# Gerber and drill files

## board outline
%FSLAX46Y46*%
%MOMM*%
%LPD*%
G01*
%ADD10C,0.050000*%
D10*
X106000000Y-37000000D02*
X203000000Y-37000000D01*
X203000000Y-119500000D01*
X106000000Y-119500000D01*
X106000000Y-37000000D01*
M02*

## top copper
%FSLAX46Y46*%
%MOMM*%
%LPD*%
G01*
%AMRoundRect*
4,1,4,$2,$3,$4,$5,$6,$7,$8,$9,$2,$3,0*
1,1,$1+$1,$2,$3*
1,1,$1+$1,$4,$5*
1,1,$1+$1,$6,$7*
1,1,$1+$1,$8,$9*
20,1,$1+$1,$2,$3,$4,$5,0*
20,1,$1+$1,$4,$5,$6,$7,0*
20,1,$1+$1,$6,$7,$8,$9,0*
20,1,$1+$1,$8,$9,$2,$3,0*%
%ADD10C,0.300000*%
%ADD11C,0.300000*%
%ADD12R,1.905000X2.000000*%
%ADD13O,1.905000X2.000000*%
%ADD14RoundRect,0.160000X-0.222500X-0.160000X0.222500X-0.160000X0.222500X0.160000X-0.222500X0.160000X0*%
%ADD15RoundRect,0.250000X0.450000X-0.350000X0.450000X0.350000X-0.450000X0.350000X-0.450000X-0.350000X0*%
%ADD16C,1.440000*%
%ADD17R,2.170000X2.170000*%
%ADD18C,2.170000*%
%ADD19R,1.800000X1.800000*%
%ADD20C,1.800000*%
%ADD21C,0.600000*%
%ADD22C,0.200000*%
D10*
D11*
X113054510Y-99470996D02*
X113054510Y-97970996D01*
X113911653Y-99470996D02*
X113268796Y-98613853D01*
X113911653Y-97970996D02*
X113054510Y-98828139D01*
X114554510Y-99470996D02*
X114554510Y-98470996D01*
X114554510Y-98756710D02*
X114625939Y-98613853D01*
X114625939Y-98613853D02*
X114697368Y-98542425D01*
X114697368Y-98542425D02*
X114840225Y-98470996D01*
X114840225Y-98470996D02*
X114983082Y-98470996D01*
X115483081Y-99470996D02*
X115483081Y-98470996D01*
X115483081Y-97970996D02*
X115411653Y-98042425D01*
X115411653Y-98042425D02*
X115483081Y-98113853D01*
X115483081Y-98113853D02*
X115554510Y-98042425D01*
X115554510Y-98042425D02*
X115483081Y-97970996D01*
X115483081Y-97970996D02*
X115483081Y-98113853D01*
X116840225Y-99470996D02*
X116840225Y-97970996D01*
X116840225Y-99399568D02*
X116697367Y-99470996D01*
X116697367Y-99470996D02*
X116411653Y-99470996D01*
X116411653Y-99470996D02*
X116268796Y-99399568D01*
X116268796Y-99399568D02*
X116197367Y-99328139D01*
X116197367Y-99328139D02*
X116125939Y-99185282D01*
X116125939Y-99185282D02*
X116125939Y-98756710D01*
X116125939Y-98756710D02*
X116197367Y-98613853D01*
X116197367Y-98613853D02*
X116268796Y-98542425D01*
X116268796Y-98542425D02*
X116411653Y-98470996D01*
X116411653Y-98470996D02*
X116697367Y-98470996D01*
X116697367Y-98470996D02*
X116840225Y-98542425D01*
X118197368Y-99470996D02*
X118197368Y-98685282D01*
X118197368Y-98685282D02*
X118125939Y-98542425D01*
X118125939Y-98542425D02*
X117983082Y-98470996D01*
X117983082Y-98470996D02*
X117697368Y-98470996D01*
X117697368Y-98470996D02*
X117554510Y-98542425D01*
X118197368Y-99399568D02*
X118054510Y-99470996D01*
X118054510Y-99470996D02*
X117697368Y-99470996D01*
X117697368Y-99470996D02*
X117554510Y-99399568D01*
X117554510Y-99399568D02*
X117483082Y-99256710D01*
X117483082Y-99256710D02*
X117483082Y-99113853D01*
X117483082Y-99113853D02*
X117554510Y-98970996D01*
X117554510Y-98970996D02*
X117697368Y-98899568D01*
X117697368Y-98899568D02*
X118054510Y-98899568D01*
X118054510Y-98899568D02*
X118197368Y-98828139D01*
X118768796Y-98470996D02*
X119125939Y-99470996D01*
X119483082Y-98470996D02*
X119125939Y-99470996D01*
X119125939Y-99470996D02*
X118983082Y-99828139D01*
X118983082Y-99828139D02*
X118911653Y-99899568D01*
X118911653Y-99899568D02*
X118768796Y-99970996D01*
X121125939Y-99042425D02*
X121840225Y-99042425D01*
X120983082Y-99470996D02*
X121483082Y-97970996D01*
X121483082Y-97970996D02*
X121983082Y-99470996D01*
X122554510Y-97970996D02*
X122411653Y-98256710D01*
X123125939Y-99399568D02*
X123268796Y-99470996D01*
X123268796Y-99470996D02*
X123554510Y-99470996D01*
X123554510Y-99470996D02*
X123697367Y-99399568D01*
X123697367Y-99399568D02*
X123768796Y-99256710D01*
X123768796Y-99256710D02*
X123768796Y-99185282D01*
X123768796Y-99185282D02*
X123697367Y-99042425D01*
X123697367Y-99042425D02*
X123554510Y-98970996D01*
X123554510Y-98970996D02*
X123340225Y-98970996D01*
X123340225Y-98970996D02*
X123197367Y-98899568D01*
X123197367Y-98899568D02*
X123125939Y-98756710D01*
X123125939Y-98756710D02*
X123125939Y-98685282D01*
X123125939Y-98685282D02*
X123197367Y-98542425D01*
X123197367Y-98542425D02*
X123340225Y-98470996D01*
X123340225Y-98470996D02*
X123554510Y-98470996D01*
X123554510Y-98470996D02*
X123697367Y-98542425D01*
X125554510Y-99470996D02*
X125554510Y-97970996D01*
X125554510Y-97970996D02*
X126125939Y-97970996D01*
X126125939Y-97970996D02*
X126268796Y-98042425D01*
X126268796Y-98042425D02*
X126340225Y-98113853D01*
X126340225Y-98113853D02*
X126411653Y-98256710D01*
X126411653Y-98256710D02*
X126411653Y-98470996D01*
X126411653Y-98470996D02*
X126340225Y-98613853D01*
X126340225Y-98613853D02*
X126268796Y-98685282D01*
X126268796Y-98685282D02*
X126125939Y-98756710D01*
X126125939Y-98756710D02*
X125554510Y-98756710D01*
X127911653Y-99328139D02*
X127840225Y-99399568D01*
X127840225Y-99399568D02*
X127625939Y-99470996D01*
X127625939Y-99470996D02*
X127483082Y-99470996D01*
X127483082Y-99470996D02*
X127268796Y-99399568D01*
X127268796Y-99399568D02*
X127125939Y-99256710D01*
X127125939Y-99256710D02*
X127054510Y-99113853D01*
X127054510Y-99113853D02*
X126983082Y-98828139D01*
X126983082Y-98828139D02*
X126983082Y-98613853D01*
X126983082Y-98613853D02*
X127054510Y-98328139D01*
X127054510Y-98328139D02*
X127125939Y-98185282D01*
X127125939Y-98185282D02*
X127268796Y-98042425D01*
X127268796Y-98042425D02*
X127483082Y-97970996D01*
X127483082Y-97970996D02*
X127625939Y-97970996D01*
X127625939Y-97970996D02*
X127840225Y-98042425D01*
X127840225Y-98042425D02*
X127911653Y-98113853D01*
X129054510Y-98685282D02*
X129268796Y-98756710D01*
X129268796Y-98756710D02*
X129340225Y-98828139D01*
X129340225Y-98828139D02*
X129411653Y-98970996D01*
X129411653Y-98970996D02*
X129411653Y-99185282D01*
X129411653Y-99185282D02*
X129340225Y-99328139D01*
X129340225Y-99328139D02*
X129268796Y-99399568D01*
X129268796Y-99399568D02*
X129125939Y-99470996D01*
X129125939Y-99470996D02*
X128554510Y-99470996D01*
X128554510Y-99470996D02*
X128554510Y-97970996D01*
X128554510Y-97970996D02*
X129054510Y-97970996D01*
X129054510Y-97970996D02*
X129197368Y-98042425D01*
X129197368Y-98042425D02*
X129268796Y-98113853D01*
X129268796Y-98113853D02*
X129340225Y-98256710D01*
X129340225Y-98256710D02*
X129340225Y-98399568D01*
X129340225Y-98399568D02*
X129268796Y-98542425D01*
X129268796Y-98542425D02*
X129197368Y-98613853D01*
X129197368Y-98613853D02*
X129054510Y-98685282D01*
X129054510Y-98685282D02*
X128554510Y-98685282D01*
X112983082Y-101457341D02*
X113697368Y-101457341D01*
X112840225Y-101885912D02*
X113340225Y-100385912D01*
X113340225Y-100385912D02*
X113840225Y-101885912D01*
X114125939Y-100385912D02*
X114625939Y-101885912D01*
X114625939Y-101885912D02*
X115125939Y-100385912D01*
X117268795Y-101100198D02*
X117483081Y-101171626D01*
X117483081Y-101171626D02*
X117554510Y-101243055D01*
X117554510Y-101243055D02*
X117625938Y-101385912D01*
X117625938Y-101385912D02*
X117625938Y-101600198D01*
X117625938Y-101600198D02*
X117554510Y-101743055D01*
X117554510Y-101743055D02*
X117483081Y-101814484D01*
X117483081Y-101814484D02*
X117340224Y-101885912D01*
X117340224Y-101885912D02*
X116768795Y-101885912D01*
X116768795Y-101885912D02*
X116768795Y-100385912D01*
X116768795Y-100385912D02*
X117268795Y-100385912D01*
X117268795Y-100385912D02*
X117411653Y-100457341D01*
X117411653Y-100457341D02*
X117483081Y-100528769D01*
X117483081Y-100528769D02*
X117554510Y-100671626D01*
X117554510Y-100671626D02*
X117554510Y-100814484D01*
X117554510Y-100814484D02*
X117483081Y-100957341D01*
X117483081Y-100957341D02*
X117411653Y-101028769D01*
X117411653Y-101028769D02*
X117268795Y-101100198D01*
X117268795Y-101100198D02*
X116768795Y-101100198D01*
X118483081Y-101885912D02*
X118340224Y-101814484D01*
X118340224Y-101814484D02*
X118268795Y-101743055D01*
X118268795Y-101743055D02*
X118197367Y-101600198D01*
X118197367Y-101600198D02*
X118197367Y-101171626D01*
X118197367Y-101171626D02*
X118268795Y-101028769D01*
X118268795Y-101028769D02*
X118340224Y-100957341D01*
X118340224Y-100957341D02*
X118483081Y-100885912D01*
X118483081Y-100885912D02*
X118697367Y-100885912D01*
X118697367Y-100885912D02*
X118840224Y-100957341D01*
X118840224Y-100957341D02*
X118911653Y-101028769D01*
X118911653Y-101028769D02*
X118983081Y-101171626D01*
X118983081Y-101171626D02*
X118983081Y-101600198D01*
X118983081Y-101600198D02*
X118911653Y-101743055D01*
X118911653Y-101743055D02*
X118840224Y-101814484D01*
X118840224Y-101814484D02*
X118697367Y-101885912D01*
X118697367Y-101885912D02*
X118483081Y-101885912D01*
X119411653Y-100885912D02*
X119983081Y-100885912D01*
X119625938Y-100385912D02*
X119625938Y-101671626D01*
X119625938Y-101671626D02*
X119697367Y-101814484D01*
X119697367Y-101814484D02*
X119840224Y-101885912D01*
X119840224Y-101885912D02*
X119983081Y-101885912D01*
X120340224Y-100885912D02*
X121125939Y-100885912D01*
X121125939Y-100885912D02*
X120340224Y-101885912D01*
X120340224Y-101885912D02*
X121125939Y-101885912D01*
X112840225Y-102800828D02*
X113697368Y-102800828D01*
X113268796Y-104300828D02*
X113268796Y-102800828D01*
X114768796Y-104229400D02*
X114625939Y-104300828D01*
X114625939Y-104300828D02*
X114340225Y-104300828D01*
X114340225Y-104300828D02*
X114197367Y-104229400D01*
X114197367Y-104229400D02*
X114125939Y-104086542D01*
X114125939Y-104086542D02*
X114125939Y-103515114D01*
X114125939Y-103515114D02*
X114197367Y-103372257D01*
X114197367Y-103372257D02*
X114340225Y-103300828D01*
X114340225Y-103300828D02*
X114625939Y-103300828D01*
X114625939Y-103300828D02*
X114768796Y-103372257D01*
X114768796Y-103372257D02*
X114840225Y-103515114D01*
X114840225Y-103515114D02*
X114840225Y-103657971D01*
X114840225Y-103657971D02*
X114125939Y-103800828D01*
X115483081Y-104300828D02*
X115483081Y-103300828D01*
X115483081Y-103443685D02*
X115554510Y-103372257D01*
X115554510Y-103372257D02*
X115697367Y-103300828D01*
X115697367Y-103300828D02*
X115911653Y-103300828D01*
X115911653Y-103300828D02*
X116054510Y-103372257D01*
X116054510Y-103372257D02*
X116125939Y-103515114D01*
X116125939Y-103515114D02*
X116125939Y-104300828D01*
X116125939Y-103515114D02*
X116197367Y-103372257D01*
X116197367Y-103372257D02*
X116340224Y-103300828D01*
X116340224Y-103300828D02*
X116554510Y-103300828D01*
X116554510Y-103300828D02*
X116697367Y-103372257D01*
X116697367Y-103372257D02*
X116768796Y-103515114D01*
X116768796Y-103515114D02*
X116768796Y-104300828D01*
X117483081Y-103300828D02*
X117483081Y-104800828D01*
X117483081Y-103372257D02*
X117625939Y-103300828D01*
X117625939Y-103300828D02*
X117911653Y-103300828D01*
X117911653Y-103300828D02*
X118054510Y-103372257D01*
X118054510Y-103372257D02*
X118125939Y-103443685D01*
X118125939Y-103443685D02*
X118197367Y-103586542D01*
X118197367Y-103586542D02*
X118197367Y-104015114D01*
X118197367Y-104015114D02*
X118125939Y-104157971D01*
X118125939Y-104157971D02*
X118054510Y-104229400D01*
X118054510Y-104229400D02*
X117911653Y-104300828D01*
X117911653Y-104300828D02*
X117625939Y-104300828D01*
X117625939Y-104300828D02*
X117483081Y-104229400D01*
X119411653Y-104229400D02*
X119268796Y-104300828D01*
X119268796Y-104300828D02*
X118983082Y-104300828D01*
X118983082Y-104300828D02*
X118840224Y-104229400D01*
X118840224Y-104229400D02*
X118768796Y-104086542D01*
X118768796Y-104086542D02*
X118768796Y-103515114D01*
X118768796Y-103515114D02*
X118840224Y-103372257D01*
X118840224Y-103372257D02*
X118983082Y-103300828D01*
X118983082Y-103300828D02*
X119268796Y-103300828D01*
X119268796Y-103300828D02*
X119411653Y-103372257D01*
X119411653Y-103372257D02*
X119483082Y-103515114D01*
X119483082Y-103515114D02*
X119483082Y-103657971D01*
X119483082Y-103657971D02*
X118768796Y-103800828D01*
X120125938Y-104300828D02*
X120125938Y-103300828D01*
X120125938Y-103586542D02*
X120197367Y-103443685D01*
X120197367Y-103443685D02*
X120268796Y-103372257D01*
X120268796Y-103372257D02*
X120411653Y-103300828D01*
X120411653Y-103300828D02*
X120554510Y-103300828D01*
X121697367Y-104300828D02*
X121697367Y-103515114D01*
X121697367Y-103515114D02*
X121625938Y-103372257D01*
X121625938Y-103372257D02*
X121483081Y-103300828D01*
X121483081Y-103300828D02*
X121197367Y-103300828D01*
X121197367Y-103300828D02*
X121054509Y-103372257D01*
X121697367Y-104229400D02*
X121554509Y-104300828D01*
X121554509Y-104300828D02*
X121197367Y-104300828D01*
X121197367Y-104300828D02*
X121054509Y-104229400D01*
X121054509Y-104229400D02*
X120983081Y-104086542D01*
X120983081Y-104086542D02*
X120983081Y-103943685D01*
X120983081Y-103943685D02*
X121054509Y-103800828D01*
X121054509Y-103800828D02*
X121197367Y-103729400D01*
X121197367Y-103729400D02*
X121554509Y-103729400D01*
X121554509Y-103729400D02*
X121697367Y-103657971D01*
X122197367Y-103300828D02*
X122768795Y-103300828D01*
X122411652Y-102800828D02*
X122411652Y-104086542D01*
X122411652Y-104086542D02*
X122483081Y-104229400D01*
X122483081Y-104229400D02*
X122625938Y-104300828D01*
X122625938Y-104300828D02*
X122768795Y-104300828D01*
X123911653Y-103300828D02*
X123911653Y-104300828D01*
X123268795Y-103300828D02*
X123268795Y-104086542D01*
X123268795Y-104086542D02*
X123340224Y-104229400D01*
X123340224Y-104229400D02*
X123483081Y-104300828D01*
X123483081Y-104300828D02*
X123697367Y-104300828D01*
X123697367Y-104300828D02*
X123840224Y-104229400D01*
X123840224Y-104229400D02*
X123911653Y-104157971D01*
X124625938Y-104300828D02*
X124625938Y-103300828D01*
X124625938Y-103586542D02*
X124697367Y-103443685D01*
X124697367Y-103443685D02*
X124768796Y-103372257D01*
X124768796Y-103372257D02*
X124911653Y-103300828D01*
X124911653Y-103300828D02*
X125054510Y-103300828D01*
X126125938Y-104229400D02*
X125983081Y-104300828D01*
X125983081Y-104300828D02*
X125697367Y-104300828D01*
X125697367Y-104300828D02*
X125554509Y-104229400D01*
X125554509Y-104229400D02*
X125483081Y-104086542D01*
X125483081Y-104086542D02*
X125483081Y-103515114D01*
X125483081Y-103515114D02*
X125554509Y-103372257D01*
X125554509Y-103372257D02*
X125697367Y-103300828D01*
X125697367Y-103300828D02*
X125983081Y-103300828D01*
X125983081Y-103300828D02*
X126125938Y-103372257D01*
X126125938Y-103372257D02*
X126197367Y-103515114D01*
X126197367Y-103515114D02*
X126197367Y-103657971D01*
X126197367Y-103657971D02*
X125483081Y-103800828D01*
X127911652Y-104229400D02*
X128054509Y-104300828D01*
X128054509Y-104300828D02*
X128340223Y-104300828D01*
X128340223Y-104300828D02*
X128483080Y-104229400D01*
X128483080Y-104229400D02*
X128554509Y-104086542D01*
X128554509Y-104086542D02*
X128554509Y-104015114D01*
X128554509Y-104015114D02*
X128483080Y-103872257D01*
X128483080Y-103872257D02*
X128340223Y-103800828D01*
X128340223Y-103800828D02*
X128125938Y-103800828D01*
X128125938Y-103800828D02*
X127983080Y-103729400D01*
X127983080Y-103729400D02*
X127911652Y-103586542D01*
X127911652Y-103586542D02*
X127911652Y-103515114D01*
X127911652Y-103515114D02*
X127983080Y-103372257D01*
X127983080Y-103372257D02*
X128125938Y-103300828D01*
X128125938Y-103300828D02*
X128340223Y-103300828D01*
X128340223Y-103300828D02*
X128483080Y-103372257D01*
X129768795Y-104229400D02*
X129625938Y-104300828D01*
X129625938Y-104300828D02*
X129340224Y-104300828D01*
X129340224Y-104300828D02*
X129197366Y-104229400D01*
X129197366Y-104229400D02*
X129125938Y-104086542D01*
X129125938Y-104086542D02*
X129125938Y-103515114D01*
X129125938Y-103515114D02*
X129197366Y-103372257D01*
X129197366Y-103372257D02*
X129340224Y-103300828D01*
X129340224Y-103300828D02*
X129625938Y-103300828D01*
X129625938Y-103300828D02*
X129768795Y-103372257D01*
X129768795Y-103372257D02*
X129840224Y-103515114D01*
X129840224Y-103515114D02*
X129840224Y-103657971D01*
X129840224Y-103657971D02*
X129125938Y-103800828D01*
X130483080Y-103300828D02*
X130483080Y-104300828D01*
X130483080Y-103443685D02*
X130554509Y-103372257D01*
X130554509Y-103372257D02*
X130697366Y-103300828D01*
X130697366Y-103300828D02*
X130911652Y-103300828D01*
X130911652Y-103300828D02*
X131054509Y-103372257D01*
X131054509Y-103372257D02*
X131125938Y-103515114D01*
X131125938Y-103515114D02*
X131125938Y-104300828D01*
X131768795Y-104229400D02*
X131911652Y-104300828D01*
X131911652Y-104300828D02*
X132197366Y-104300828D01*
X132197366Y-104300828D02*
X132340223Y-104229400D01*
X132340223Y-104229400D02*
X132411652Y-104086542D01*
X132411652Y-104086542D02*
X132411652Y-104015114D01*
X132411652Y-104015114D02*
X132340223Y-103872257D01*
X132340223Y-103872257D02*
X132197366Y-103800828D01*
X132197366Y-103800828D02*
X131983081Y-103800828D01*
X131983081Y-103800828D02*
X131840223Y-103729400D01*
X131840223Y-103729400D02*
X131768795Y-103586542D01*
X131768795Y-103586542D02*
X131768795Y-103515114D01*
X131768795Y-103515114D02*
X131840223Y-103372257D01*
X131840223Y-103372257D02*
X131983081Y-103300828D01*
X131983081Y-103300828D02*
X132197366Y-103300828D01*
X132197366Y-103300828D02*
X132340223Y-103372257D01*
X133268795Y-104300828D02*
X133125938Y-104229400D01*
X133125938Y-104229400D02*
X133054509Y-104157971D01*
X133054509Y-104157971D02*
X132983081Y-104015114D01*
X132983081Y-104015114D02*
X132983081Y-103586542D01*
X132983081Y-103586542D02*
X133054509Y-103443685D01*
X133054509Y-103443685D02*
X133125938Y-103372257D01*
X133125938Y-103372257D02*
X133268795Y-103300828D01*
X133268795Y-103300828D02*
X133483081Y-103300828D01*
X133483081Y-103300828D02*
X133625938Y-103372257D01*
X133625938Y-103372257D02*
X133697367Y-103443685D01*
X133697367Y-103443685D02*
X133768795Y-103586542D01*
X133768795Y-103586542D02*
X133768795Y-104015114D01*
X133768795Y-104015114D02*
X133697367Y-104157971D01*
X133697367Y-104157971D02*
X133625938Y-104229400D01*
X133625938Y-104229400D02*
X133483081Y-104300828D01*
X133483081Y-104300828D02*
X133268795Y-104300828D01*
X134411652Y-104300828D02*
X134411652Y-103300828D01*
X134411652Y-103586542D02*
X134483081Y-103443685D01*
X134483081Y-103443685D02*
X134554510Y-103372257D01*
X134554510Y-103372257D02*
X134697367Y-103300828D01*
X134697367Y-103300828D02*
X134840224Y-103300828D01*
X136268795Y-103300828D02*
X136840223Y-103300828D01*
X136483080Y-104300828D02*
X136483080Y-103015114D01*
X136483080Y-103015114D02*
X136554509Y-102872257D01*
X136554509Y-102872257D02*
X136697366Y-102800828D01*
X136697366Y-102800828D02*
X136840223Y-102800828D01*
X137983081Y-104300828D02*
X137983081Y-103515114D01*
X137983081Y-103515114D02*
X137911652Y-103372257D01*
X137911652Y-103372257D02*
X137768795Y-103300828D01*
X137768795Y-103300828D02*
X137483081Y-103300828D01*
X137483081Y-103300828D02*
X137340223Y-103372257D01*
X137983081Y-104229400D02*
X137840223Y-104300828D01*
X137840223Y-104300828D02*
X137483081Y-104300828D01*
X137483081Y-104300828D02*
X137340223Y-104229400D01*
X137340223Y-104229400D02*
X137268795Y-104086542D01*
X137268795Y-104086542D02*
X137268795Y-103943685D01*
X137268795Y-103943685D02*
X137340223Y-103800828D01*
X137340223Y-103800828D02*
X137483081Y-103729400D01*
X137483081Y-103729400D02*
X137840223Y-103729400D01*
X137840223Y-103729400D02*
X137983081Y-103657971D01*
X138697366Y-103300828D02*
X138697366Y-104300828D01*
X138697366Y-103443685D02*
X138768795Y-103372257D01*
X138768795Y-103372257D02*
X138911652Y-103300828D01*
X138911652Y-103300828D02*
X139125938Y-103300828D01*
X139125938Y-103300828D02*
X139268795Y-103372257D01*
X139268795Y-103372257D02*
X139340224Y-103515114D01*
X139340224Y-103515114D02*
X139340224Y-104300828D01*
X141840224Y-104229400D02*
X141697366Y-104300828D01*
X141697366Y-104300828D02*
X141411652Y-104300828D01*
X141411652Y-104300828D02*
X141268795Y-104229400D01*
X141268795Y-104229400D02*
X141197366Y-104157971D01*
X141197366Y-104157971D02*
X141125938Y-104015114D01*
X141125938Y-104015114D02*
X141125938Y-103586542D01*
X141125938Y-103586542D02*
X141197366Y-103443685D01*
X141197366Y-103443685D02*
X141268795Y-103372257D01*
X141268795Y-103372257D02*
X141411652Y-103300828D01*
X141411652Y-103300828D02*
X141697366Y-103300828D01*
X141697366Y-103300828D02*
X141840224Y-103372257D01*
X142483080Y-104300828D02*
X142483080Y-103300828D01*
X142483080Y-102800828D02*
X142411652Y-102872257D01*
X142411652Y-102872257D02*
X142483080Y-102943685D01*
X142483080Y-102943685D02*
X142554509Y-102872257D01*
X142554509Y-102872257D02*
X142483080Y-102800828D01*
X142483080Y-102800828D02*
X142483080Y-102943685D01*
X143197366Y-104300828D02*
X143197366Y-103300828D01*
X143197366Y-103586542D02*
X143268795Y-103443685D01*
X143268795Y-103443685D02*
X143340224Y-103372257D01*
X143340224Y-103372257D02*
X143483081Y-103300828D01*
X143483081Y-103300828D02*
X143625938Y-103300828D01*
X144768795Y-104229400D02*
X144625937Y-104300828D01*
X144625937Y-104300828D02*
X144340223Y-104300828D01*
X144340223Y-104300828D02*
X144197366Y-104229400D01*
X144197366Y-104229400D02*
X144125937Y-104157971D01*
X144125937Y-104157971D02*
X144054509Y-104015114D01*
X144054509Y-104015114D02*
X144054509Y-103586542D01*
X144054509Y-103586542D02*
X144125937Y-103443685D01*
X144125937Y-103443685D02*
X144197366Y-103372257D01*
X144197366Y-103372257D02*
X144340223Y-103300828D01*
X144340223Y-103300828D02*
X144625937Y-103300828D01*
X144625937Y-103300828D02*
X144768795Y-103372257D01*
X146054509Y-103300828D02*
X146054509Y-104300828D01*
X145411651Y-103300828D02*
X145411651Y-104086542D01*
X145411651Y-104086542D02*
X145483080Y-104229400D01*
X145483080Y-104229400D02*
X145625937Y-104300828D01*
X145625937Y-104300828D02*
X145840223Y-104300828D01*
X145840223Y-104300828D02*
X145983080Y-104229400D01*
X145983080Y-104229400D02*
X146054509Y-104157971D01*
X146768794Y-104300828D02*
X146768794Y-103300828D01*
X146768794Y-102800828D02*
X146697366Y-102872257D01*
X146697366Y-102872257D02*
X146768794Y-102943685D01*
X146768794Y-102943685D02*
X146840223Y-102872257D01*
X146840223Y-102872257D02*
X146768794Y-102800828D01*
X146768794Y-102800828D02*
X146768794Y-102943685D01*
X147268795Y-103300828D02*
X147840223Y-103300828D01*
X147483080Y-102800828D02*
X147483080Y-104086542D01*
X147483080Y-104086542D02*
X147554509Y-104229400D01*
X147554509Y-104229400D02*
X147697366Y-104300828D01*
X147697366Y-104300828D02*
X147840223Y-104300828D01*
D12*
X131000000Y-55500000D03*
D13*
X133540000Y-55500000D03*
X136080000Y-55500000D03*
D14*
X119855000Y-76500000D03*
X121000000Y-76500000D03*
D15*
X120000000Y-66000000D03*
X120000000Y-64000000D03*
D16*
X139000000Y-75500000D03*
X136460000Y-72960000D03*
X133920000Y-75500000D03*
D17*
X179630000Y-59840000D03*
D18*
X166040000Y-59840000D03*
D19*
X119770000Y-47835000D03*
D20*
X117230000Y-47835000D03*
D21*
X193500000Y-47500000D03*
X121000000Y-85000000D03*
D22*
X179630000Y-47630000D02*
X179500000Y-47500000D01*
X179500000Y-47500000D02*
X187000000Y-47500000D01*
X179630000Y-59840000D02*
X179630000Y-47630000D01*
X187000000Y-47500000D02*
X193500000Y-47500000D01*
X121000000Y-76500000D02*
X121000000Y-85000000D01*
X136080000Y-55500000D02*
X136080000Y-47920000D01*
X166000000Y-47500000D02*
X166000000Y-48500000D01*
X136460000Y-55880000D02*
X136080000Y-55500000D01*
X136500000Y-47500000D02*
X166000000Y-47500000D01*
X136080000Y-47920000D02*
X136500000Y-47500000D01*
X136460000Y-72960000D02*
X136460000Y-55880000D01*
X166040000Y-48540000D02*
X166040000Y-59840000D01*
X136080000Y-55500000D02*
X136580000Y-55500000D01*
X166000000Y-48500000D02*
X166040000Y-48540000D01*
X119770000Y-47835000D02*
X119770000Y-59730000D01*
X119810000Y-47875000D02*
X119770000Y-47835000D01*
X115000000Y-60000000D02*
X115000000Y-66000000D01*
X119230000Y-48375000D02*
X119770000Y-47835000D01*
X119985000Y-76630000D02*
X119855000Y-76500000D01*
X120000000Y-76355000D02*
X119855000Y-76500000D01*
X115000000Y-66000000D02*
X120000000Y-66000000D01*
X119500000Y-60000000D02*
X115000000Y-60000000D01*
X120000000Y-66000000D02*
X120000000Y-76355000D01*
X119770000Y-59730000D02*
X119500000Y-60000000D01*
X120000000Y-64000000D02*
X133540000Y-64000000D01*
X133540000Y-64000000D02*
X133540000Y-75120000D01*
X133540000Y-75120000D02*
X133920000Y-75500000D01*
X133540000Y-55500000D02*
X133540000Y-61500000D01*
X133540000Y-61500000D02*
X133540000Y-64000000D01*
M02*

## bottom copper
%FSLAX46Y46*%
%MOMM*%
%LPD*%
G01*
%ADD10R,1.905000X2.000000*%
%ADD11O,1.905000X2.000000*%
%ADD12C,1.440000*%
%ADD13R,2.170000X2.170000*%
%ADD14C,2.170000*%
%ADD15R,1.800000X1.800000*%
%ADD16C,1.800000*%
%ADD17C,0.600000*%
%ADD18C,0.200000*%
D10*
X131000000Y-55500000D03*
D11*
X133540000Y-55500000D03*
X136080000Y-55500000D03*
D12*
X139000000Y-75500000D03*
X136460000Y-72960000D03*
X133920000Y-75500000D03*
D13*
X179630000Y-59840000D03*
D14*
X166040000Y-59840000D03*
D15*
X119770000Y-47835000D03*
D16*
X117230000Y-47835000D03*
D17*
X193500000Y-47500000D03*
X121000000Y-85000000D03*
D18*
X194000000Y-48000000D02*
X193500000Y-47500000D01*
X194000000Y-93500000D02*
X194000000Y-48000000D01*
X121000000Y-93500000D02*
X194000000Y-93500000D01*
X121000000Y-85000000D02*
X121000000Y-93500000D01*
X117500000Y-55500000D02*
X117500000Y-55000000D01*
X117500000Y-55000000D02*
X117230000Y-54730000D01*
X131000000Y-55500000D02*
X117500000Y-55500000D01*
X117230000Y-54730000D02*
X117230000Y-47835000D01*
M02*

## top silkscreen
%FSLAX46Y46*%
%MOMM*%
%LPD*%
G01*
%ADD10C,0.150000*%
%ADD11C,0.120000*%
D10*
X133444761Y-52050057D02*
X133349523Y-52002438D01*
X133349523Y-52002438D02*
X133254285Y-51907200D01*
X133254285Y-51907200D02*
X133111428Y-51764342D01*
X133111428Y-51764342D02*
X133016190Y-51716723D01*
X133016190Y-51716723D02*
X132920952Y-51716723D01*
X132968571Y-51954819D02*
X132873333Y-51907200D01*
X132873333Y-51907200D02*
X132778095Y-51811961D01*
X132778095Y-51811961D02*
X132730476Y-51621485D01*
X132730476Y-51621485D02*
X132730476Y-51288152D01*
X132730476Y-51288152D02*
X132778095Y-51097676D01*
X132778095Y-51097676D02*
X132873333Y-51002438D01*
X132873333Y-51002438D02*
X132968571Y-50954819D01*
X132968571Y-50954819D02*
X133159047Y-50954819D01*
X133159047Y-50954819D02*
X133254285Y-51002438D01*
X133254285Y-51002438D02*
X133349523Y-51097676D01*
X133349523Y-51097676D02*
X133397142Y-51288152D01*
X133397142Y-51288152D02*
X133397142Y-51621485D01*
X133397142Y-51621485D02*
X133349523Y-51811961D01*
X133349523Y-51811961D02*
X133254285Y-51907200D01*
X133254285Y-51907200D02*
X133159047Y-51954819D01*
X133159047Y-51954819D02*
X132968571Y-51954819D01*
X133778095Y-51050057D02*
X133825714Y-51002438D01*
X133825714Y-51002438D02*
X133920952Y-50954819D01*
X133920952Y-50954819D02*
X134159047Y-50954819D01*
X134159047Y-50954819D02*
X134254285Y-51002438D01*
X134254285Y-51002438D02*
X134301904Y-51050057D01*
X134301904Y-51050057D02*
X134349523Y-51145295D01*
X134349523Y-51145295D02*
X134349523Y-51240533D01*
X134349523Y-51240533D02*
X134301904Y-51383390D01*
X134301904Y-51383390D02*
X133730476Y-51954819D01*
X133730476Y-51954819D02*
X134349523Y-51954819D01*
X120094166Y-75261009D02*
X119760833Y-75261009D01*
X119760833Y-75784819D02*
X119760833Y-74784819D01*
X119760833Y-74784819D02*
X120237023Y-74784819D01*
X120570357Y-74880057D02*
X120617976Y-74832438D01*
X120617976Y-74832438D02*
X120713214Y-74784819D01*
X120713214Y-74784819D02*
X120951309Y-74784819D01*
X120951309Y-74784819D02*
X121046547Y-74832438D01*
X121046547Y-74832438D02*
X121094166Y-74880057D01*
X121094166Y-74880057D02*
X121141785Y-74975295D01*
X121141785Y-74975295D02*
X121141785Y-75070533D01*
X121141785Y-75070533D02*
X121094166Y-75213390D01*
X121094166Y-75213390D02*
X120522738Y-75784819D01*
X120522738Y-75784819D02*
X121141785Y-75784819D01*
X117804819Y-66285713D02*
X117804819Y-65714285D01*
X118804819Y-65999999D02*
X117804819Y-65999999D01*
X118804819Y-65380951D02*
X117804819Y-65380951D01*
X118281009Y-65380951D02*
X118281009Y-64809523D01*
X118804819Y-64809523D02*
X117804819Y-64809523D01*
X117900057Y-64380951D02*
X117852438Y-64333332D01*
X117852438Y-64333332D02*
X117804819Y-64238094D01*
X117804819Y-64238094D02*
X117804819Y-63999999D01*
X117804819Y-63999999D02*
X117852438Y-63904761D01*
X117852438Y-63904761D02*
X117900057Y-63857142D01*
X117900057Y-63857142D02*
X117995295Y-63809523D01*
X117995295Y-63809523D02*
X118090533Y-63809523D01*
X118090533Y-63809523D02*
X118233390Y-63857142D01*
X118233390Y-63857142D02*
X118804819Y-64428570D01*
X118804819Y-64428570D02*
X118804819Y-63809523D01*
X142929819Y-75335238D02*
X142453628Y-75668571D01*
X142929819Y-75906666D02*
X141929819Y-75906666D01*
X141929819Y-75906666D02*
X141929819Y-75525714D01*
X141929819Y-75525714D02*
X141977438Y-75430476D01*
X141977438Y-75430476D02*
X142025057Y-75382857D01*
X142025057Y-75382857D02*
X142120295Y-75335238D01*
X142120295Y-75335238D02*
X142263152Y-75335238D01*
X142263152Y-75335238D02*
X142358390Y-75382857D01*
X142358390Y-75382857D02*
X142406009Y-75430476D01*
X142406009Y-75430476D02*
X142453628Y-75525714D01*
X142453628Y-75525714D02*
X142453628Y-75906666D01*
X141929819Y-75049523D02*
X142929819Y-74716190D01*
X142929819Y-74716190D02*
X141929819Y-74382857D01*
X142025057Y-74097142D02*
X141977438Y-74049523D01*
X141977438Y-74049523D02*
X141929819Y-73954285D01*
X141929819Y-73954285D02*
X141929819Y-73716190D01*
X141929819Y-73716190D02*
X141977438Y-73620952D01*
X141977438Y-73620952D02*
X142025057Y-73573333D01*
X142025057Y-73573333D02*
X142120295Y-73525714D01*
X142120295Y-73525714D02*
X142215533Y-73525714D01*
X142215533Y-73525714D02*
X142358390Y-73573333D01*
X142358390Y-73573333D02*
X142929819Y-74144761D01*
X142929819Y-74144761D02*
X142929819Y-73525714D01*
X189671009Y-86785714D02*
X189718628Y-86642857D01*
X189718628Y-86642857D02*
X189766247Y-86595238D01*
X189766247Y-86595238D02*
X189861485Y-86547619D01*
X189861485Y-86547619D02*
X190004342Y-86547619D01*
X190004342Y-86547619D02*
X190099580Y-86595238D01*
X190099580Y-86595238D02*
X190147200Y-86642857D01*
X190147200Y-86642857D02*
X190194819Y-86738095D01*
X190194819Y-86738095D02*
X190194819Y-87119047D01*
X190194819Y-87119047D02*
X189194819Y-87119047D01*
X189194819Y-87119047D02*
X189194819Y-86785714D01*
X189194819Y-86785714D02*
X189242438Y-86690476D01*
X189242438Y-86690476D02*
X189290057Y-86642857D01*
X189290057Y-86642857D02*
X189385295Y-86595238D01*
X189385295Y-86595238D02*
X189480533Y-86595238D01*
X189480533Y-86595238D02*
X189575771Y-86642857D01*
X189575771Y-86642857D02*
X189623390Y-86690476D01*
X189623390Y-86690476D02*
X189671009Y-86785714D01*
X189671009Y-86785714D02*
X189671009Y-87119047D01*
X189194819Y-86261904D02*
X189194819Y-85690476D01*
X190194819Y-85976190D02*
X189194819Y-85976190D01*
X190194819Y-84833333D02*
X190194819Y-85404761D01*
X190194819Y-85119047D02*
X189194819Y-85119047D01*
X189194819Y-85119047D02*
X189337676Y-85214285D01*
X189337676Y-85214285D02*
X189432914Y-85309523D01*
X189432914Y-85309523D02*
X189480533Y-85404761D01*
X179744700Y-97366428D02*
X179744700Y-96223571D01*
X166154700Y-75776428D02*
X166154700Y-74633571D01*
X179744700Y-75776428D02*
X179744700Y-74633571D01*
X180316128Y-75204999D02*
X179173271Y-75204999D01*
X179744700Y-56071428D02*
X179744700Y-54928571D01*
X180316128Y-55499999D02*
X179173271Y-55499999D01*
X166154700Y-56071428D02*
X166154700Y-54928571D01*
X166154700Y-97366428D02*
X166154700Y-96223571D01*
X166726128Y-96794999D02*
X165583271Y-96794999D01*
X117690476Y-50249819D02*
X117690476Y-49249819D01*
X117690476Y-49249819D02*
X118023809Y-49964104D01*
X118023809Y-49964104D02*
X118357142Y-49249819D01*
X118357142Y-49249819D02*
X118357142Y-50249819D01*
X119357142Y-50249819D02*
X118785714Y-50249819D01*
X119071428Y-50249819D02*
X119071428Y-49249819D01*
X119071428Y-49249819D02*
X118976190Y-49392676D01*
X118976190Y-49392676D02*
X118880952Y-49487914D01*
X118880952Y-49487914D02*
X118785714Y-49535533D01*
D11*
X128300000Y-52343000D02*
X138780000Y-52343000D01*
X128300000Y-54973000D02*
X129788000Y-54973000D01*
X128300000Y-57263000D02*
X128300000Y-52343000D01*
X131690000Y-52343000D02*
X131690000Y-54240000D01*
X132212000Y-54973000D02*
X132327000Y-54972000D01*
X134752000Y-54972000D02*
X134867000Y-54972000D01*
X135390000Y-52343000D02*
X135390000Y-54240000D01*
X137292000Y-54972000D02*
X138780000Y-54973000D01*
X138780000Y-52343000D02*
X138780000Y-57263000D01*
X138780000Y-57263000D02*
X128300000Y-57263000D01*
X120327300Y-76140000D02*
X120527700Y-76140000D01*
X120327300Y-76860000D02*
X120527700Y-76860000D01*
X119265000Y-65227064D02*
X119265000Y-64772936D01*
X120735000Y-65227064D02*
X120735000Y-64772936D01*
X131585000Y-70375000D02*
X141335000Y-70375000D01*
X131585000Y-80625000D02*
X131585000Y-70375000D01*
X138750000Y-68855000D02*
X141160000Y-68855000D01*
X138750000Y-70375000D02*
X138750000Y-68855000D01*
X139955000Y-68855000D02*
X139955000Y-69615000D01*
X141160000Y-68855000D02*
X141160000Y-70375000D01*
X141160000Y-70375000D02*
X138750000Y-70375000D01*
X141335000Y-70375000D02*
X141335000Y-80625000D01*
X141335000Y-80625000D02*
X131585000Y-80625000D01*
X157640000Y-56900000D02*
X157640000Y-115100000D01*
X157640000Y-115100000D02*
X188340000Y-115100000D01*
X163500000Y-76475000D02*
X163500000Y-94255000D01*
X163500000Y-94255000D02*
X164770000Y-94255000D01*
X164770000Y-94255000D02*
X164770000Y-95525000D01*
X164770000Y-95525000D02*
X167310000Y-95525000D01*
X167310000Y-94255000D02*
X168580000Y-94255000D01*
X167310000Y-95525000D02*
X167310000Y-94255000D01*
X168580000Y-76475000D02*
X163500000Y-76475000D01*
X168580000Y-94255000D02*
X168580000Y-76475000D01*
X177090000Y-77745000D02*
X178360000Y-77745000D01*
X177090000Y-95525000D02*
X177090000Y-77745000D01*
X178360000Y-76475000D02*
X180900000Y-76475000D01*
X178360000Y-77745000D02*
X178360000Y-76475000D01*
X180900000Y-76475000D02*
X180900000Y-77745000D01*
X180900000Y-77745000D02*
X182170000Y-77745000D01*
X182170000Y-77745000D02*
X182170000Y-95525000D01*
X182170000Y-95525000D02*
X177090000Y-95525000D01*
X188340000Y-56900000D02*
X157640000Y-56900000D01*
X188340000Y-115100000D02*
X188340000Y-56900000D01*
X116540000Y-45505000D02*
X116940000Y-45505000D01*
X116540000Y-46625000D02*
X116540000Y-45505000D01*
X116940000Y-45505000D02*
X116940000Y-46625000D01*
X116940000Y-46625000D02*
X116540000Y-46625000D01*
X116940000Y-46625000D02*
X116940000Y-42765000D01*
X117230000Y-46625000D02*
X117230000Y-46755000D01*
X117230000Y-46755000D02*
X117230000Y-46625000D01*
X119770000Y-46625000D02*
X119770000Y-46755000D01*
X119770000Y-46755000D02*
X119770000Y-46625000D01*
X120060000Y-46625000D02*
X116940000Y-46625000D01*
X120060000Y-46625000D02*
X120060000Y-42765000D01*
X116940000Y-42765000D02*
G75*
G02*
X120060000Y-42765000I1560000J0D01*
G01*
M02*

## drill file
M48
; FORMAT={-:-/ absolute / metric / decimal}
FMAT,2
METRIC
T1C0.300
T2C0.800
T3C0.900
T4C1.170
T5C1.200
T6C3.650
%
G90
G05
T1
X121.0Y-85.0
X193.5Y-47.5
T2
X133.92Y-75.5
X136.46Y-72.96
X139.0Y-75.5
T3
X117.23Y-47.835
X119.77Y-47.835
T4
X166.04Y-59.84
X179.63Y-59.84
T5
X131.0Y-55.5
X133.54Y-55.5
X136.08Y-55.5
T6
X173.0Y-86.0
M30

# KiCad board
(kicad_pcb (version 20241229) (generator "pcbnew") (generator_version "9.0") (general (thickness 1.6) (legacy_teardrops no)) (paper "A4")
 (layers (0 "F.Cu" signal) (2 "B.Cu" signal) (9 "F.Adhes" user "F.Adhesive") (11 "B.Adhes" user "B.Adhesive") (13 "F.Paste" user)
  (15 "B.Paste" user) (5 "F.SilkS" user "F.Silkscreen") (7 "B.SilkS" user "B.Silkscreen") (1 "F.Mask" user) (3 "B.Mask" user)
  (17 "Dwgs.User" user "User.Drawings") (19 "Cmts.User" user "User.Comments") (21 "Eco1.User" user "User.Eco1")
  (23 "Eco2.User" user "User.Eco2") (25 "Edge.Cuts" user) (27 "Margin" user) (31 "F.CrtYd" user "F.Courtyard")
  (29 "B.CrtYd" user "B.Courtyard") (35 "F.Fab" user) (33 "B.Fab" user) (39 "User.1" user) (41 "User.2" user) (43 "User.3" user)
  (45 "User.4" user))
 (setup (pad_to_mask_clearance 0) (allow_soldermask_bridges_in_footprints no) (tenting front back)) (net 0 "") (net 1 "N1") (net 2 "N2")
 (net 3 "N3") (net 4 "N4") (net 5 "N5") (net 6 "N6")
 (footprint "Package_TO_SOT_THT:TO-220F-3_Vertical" (layer "F.Cu") (at 131 55.5)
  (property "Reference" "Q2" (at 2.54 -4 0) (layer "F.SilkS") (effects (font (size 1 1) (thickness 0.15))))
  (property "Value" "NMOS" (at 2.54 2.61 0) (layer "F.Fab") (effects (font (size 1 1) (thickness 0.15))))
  (fp_line (start -2.7 -3.157) (end 7.78 -3.157) (stroke (width 0.12) (type solid)) (layer "F.SilkS"))
  (fp_line (start -2.7 -0.527) (end -1.212 -0.527) (stroke (width 0.12) (type solid)) (layer "F.SilkS"))
  (fp_line (start -2.7 1.763) (end -2.7 -3.157) (stroke (width 0.12) (type solid)) (layer "F.SilkS"))
  (fp_line (start 0.69 -3.157) (end 0.69 -1.26) (stroke (width 0.12) (type solid)) (layer "F.SilkS"))
  (fp_line (start 1.212 -0.527) (end 1.327 -0.528) (stroke (width 0.12) (type solid)) (layer "F.SilkS"))
  (fp_line (start 3.752 -0.528) (end 3.867 -0.528) (stroke (width 0.12) (type solid)) (layer "F.SilkS"))
  (fp_line (start 4.39 -3.157) (end 4.39 -1.26) (stroke (width 0.12) (type solid)) (layer "F.SilkS"))
  (fp_line (start 6.292 -0.528) (end 7.78 -0.527) (stroke (width 0.12) (type solid)) (layer "F.SilkS"))
  (fp_line (start 7.78 -3.157) (end 7.78 1.763) (stroke (width 0.12) (type solid)) (layer "F.SilkS"))
  (fp_line (start 7.78 1.763) (end -2.7 1.763) (stroke (width 0.12) (type solid)) (layer "F.SilkS"))
  (pad "1" thru_hole rect (at 0 0) (size 1.905 2) (drill 1.2) (layers "*.Cu" "*.Mask") (remove_unused_layers no) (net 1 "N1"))
  (pad "2" thru_hole oval (at 2.54 0) (size 1.905 2) (drill 1.2) (layers "*.Cu" "*.Mask") (remove_unused_layers no) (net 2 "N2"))
  (pad "3" thru_hole oval (at 5.08 0) (size 1.905 2) (drill 1.2) (layers "*.Cu" "*.Mask") (remove_unused_layers no) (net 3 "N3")))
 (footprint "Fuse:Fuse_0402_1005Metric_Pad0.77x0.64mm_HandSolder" (layer "F.Cu") (at 120.4275 76.5)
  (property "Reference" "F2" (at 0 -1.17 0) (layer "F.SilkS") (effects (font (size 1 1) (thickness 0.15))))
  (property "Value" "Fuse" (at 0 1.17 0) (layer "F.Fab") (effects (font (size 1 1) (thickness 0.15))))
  (fp_line (start -0.1002 -0.36) (end 0.1002 -0.36) (stroke (width 0.12) (type solid)) (layer "F.SilkS"))
  (fp_line (start -0.1002 0.36) (end 0.1002 0.36) (stroke (width 0.12) (type solid)) (layer "F.SilkS"))
  (pad "1" smd roundrect (at -0.5725 0) (size 0.765 0.64) (layers "F.Cu" "F.Mask" "F.Paste") (roundrect_rratio 0.25) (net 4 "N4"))
  (pad "2" smd roundrect (at 0.5725 0) (size 0.765 0.64) (layers "F.Cu" "F.Mask" "F.Paste") (roundrect_rratio 0.25) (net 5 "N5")))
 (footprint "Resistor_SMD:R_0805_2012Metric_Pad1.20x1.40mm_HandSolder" (layer "F.Cu") (at 120 65 90)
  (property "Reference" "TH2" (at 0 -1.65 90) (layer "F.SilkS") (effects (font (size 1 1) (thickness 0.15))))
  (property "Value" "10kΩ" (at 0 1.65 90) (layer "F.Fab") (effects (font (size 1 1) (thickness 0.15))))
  (fp_line (start -0.227064 -0.735) (end 0.227064 -0.735) (stroke (width 0.12) (type solid)) (layer "F.SilkS"))
  (fp_line (start -0.227064 0.735) (end 0.227064 0.735) (stroke (width 0.12) (type solid)) (layer "F.SilkS"))
  (pad "1" smd roundrect (at -1 0 90) (size 1.2 1.4) (layers "F.Cu" "F.Mask" "F.Paste") (roundrect_rratio 0.208333) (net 4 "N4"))
  (pad "2" smd roundrect (at 1 0 90) (size 1.2 1.4) (layers "F.Cu" "F.Mask" "F.Paste") (roundrect_rratio 0.208333) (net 2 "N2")))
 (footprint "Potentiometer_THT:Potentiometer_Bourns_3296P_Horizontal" (layer "F.Cu") (at 139 75.5 -90)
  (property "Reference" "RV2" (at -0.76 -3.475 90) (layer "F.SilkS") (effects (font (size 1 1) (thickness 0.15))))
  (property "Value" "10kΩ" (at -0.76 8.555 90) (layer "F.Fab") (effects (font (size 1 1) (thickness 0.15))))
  (fp_line (start -5.125 7.415) (end -5.125 -2.335) (stroke (width 0.12) (type solid)) (layer "F.SilkS"))
  (fp_line (start 5.125 7.415) (end -5.125 7.415) (stroke (width 0.12) (type solid)) (layer "F.SilkS"))
  (fp_line (start -6.645 0.25) (end -6.645 -2.16) (stroke (width 0.12) (type solid)) (layer "F.SilkS"))
  (fp_line (start -5.125 0.25) (end -6.645 0.25) (stroke (width 0.12) (type solid)) (layer "F.SilkS"))
  (fp_line (start -6.645 -0.955) (end -5.885 -0.955) (stroke (width 0.12) (type solid)) (layer "F.SilkS"))
  (fp_line (start -6.645 -2.16) (end -5.125 -2.16) (stroke (width 0.12) (type solid)) (layer "F.SilkS"))
  (fp_line (start -5.125 -2.16) (end -5.125 0.25) (stroke (width 0.12) (type solid)) (layer "F.SilkS"))
  (fp_line (start -5.125 -2.335) (end 5.125 -2.335) (stroke (width 0.12) (type solid)) (layer "F.SilkS"))
  (fp_line (start 5.125 -2.335) (end 5.125 7.415) (stroke (width 0.12) (type solid)) (layer "F.SilkS"))
  (pad "1" thru_hole circle (at 0 0 270) (size 1.44 1.44) (drill 0.8) (layers "*.Cu" "*.Mask") (remove_unused_layers no) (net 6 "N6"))
  (pad "2" thru_hole circle (at -2.54 2.54 270) (size 1.44 1.44) (drill 0.8) (layers "*.Cu" "*.Mask") (remove_unused_layers no) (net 3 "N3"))
  (pad "3" thru_hole circle (at 0 5.08 270) (size 1.44 1.44) (drill 0.8) (layers "*.Cu" "*.Mask") (remove_unused_layers no) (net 2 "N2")))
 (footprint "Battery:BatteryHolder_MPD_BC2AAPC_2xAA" (layer "F.Cu") (at 179.63 59.84 -90)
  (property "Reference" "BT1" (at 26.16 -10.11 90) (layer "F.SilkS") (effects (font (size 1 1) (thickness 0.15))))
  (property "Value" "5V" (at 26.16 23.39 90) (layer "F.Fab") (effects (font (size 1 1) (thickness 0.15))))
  (fp_line (start -2.94 21.99) (end 55.26 21.99) (stroke (width 0.12) (type solid)) (layer "F.SilkS"))
  (fp_line (start 55.26 21.99) (end 55.26 -8.71) (stroke (width 0.12) (type solid)) (layer "F.SilkS"))
  (fp_line (start 16.635 16.13) (end 34.415 16.13) (stroke (width 0.12) (type solid)) (layer "F.SilkS"))
  (fp_line (start 34.415 16.13) (end 34.415 14.86) (stroke (width 0.12) (type solid)) (layer "F.SilkS"))
  (fp_line (start 34.415 14.86) (end 35.685 14.86) (stroke (width 0.12) (type solid)) (layer "F.SilkS"))
  (fp_line (start 35.685 14.86) (end 35.685 12.32) (stroke (width 0.12) (type solid)) (layer "F.SilkS"))
  (fp_line (start 34.415 12.32) (end 34.415 11.05) (stroke (width 0.12) (type solid)) (layer "F.SilkS"))
  (fp_line (start 35.685 12.32) (end 34.415 12.32) (stroke (width 0.12) (type solid)) (layer "F.SilkS"))
  (fp_line (start 16.635 11.05) (end 16.635 16.13) (stroke (width 0.12) (type solid)) (layer "F.SilkS"))
  (fp_line (start 34.415 11.05) (end 16.635 11.05) (stroke (width 0.12) (type solid)) (layer "F.SilkS"))
  (fp_line (start 17.905 2.54) (end 17.905 1.27) (stroke (width 0.12) (type solid)) (layer "F.SilkS"))
  (fp_line (start 35.685 2.54) (end 17.905 2.54) (stroke (width 0.12) (type solid)) (layer "F.SilkS"))
  (fp_line (start 16.635 1.27) (end 16.635 -1.27) (stroke (width 0.12) (type solid)) (layer "F.SilkS"))
  (fp_line (start 17.905 1.27) (end 16.635 1.27) (stroke (width 0.12) (type solid)) (layer "F.SilkS"))
  (fp_line (start 16.635 -1.27) (end 17.905 -1.27) (stroke (width 0.12) (type solid)) (layer "F.SilkS"))
  (fp_line (start 17.905 -1.27) (end 17.905 -2.54) (stroke (width 0.12) (type solid)) (layer "F.SilkS"))
  (fp_line (start 17.905 -2.54) (end 35.685 -2.54) (stroke (width 0.12) (type solid)) (layer "F.SilkS"))
  (fp_line (start 35.685 -2.54) (end 35.685 2.54) (stroke (width 0.12) (type solid)) (layer "F.SilkS"))
  (fp_line (start -2.94 -8.71) (end -2.94 21.99) (stroke (width 0.12) (type solid)) (layer "F.SilkS"))
  (fp_line (start 55.26 -8.71) (end -2.94 -8.71) (stroke (width 0.12) (type solid)) (layer "F.SilkS"))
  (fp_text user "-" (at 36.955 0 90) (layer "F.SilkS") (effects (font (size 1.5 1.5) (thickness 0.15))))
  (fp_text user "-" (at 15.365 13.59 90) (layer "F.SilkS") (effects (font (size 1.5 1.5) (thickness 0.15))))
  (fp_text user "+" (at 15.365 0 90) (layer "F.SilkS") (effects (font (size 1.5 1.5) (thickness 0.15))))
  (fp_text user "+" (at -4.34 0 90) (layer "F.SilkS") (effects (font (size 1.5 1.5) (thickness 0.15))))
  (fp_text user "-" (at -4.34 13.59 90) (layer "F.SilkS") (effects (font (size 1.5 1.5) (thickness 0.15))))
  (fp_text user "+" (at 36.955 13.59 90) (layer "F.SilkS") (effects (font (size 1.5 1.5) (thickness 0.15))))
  (pad "" np_thru_hole circle (at 26.16 6.63 270) (size 3.65 3.65) (drill 3.65) (layers "*.Cu" "*.Mask"))
  (pad "1" thru_hole rect (at 0 0 270) (size 2.17 2.17) (drill 1.17) (layers "*.Cu" "*.Mask") (remove_unused_layers no) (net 5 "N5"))
  (pad "2" thru_hole circle (at 0 13.59 270) (size 2.17 2.17) (drill 1.17) (layers "*.Cu" "*.Mask") (remove_unused_layers no) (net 3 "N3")))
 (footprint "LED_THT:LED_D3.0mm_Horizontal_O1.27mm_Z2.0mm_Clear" (layer "F.Cu") (at 119.77 47.835 180)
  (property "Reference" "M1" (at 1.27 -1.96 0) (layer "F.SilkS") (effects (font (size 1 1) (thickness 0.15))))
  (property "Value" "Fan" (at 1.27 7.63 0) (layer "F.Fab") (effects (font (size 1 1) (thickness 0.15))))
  (fp_line (start 3.23 2.33) (end 2.83 2.33) (stroke (width 0.12) (type solid)) (layer "F.SilkS"))
  (fp_line (start 3.23 1.21) (end 3.23 2.33) (stroke (width 0.12) (type solid)) (layer "F.SilkS"))
  (fp_line (start 2.83 2.33) (end 2.83 1.21) (stroke (width 0.12) (type solid)) (layer "F.SilkS"))
  (fp_line (start 2.83 1.21) (end 3.23 1.21) (stroke (width 0.12) (type solid)) (layer "F.SilkS"))
  (fp_line (start 2.83 1.21) (end 2.83 5.07) (stroke (width 0.12) (type solid)) (layer "F.SilkS"))
  (fp_line (start 2.54 1.21) (end 2.54 1.08) (stroke (width 0.12) (type solid)) (layer "F.SilkS"))
  (fp_line (start 2.54 1.08) (end 2.54 1.21) (stroke (width 0.12) (type solid)) (layer "F.SilkS"))
  (fp_line (start 0 1.21) (end 0 1.08) (stroke (width 0.12) (type solid)) (layer "F.SilkS"))
  (fp_line (start 0 1.08) (end 0 1.21) (stroke (width 0.12) (type solid)) (layer "F.SilkS"))
  (fp_line (start -0.29 1.21) (end 2.83 1.21) (stroke (width 0.12) (type solid)) (layer "F.SilkS"))
  (fp_line (start -0.29 1.21) (end -0.29 5.07) (stroke (width 0.12) (type solid)) (layer "F.SilkS"))
  (fp_arc (start 2.83 5.07) (mid 1.27 6.63) (end -0.29 5.07) (stroke (width 0.12) (type solid)) (layer "F.SilkS"))
  (pad "1" thru_hole rect (at 0 0 180) (size 1.8 1.8) (drill 0.9) (layers "*.Cu" "*.Mask") (remove_unused_layers no) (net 4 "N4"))
  (pad "2" thru_hole circle (at 2.54 0 180) (size 1.8 1.8) (drill 0.9) (layers "*.Cu" "*.Mask") (remove_unused_layers no) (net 1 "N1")))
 (gr_rect (start 106 37) (end 203 119.5) (stroke (width 0.05) (type default)) (fill no) (layer "Edge.Cuts"))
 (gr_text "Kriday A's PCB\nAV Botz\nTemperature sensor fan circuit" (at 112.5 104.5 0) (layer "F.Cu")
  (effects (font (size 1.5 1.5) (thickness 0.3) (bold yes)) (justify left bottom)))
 (segment (start 179.63 47.63) (end 179.5 47.5) (width 0.2) (layer "F.Cu") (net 5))
 (segment (start 179.5 47.5) (end 187 47.5) (width 0.2) (layer "F.Cu") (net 5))
 (segment (start 179.63 59.84) (end 179.63 47.63) (width 0.2) (layer "F.Cu") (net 5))
 (segment (start 187 47.5) (end 193.5 47.5) (width 0.2) (layer "F.Cu") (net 5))
 (segment (start 121 76.5) (end 121 85) (width 0.2) (layer "F.Cu") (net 5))
 (via (at 193.5 47.5) (size 0.6) (drill 0.3) (layers "F.Cu" "B.Cu") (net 5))
 (via (at 121 85) (size 0.6) (drill 0.3) (layers "F.Cu" "B.Cu") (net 5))
 (segment (start 194 48) (end 193.5 47.5) (width 0.2) (layer "B.Cu") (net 5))
 (segment (start 194 93.5) (end 194 48) (width 0.2) (layer "B.Cu") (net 5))
 (segment (start 121 93.5) (end 194 93.5) (width 0.2) (layer "B.Cu") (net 5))
 (segment (start 121 85) (end 121 93.5) (width 0.2) (layer "B.Cu") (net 5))
 (segment (start 136.08 55.5) (end 136.08 47.92) (width 0.2) (layer "F.Cu") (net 3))
 (segment (start 166 47.5) (end 166 48.5) (width 0.2) (layer "F.Cu") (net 3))
 (segment (start 136.46 55.88) (end 136.08 55.5) (width 0.2) (layer "F.Cu") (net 3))
 (segment (start 136.5 47.5) (end 166 47.5) (width 0.2) (layer "F.Cu") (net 3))
 (segment (start 136.08 47.92) (end 136.5 47.5) (width 0.2) (layer "F.Cu") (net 3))
 (segment (start 136.46 72.96) (end 136.46 55.88) (width 0.2) (layer "F.Cu") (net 3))
 (segment (start 166.04 48.54) (end 166.04 59.84) (width 0.2) (layer "F.Cu") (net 3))
 (segment (start 136.08 55.5) (end 136.58 55.5) (width 0.2) (layer "F.Cu") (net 3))
 (segment (start 166 48.5) (end 166.04 48.54) (width 0.2) (layer "F.Cu") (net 3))
 (segment (start 119.77 47.835) (end 119.77 59.73) (width 0.2) (layer "F.Cu") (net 4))
 (segment (start 119.81 47.875) (end 119.77 47.835) (width 0.2) (layer "F.Cu") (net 4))
 (segment (start 115 60) (end 115 66) (width 0.2) (layer "F.Cu") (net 4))
 (segment (start 119.23 48.375) (end 119.77 47.835) (width 0.2) (layer "F.Cu") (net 4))
 (segment (start 119.985 76.63) (end 119.855 76.5) (width 0.2) (layer "F.Cu") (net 4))
 (segment (start 120 76.355) (end 119.855 76.5) (width 0.2) (layer "F.Cu") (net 4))
 (segment (start 115 66) (end 120 66) (width 0.2) (layer "F.Cu") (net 4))
 (segment (start 119.5 60) (end 115 60) (width 0.2) (layer "F.Cu") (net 4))
 (segment (start 120 66) (end 120 76.355) (width 0.2) (layer "F.Cu") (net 4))
 (segment (start 119.77 59.73) (end 119.5 60) (width 0.2) (layer "F.Cu") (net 4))
 (segment (start 120 64) (end 133.54 64) (width 0.2) (layer "F.Cu") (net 2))
 (segment (start 133.54 64) (end 133.54 75.12) (width 0.2) (layer "F.Cu") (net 2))
 (segment (start 133.54 75.12) (end 133.92 75.5) (width 0.2) (layer "F.Cu") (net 2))
 (segment (start 133.54 55.5) (end 133.54 61.5) (width 0.2) (layer "F.Cu") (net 2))
 (segment (start 133.54 61.5) (end 133.54 64) (width 0.2) (layer "F.Cu") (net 2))
 (segment (start 117.5 55.5) (end 117.5 55) (width 0.2) (layer "B.Cu") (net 1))
 (segment (start 117.5 55) (end 117.23 54.73) (width 0.2) (layer "B.Cu") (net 1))
 (segment (start 131 55.5) (end 117.5 55.5) (width 0.2) (layer "B.Cu") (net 1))
 (segment (start 117.23 54.73) (end 117.23 47.835) (width 0.2) (layer "B.Cu") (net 1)))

